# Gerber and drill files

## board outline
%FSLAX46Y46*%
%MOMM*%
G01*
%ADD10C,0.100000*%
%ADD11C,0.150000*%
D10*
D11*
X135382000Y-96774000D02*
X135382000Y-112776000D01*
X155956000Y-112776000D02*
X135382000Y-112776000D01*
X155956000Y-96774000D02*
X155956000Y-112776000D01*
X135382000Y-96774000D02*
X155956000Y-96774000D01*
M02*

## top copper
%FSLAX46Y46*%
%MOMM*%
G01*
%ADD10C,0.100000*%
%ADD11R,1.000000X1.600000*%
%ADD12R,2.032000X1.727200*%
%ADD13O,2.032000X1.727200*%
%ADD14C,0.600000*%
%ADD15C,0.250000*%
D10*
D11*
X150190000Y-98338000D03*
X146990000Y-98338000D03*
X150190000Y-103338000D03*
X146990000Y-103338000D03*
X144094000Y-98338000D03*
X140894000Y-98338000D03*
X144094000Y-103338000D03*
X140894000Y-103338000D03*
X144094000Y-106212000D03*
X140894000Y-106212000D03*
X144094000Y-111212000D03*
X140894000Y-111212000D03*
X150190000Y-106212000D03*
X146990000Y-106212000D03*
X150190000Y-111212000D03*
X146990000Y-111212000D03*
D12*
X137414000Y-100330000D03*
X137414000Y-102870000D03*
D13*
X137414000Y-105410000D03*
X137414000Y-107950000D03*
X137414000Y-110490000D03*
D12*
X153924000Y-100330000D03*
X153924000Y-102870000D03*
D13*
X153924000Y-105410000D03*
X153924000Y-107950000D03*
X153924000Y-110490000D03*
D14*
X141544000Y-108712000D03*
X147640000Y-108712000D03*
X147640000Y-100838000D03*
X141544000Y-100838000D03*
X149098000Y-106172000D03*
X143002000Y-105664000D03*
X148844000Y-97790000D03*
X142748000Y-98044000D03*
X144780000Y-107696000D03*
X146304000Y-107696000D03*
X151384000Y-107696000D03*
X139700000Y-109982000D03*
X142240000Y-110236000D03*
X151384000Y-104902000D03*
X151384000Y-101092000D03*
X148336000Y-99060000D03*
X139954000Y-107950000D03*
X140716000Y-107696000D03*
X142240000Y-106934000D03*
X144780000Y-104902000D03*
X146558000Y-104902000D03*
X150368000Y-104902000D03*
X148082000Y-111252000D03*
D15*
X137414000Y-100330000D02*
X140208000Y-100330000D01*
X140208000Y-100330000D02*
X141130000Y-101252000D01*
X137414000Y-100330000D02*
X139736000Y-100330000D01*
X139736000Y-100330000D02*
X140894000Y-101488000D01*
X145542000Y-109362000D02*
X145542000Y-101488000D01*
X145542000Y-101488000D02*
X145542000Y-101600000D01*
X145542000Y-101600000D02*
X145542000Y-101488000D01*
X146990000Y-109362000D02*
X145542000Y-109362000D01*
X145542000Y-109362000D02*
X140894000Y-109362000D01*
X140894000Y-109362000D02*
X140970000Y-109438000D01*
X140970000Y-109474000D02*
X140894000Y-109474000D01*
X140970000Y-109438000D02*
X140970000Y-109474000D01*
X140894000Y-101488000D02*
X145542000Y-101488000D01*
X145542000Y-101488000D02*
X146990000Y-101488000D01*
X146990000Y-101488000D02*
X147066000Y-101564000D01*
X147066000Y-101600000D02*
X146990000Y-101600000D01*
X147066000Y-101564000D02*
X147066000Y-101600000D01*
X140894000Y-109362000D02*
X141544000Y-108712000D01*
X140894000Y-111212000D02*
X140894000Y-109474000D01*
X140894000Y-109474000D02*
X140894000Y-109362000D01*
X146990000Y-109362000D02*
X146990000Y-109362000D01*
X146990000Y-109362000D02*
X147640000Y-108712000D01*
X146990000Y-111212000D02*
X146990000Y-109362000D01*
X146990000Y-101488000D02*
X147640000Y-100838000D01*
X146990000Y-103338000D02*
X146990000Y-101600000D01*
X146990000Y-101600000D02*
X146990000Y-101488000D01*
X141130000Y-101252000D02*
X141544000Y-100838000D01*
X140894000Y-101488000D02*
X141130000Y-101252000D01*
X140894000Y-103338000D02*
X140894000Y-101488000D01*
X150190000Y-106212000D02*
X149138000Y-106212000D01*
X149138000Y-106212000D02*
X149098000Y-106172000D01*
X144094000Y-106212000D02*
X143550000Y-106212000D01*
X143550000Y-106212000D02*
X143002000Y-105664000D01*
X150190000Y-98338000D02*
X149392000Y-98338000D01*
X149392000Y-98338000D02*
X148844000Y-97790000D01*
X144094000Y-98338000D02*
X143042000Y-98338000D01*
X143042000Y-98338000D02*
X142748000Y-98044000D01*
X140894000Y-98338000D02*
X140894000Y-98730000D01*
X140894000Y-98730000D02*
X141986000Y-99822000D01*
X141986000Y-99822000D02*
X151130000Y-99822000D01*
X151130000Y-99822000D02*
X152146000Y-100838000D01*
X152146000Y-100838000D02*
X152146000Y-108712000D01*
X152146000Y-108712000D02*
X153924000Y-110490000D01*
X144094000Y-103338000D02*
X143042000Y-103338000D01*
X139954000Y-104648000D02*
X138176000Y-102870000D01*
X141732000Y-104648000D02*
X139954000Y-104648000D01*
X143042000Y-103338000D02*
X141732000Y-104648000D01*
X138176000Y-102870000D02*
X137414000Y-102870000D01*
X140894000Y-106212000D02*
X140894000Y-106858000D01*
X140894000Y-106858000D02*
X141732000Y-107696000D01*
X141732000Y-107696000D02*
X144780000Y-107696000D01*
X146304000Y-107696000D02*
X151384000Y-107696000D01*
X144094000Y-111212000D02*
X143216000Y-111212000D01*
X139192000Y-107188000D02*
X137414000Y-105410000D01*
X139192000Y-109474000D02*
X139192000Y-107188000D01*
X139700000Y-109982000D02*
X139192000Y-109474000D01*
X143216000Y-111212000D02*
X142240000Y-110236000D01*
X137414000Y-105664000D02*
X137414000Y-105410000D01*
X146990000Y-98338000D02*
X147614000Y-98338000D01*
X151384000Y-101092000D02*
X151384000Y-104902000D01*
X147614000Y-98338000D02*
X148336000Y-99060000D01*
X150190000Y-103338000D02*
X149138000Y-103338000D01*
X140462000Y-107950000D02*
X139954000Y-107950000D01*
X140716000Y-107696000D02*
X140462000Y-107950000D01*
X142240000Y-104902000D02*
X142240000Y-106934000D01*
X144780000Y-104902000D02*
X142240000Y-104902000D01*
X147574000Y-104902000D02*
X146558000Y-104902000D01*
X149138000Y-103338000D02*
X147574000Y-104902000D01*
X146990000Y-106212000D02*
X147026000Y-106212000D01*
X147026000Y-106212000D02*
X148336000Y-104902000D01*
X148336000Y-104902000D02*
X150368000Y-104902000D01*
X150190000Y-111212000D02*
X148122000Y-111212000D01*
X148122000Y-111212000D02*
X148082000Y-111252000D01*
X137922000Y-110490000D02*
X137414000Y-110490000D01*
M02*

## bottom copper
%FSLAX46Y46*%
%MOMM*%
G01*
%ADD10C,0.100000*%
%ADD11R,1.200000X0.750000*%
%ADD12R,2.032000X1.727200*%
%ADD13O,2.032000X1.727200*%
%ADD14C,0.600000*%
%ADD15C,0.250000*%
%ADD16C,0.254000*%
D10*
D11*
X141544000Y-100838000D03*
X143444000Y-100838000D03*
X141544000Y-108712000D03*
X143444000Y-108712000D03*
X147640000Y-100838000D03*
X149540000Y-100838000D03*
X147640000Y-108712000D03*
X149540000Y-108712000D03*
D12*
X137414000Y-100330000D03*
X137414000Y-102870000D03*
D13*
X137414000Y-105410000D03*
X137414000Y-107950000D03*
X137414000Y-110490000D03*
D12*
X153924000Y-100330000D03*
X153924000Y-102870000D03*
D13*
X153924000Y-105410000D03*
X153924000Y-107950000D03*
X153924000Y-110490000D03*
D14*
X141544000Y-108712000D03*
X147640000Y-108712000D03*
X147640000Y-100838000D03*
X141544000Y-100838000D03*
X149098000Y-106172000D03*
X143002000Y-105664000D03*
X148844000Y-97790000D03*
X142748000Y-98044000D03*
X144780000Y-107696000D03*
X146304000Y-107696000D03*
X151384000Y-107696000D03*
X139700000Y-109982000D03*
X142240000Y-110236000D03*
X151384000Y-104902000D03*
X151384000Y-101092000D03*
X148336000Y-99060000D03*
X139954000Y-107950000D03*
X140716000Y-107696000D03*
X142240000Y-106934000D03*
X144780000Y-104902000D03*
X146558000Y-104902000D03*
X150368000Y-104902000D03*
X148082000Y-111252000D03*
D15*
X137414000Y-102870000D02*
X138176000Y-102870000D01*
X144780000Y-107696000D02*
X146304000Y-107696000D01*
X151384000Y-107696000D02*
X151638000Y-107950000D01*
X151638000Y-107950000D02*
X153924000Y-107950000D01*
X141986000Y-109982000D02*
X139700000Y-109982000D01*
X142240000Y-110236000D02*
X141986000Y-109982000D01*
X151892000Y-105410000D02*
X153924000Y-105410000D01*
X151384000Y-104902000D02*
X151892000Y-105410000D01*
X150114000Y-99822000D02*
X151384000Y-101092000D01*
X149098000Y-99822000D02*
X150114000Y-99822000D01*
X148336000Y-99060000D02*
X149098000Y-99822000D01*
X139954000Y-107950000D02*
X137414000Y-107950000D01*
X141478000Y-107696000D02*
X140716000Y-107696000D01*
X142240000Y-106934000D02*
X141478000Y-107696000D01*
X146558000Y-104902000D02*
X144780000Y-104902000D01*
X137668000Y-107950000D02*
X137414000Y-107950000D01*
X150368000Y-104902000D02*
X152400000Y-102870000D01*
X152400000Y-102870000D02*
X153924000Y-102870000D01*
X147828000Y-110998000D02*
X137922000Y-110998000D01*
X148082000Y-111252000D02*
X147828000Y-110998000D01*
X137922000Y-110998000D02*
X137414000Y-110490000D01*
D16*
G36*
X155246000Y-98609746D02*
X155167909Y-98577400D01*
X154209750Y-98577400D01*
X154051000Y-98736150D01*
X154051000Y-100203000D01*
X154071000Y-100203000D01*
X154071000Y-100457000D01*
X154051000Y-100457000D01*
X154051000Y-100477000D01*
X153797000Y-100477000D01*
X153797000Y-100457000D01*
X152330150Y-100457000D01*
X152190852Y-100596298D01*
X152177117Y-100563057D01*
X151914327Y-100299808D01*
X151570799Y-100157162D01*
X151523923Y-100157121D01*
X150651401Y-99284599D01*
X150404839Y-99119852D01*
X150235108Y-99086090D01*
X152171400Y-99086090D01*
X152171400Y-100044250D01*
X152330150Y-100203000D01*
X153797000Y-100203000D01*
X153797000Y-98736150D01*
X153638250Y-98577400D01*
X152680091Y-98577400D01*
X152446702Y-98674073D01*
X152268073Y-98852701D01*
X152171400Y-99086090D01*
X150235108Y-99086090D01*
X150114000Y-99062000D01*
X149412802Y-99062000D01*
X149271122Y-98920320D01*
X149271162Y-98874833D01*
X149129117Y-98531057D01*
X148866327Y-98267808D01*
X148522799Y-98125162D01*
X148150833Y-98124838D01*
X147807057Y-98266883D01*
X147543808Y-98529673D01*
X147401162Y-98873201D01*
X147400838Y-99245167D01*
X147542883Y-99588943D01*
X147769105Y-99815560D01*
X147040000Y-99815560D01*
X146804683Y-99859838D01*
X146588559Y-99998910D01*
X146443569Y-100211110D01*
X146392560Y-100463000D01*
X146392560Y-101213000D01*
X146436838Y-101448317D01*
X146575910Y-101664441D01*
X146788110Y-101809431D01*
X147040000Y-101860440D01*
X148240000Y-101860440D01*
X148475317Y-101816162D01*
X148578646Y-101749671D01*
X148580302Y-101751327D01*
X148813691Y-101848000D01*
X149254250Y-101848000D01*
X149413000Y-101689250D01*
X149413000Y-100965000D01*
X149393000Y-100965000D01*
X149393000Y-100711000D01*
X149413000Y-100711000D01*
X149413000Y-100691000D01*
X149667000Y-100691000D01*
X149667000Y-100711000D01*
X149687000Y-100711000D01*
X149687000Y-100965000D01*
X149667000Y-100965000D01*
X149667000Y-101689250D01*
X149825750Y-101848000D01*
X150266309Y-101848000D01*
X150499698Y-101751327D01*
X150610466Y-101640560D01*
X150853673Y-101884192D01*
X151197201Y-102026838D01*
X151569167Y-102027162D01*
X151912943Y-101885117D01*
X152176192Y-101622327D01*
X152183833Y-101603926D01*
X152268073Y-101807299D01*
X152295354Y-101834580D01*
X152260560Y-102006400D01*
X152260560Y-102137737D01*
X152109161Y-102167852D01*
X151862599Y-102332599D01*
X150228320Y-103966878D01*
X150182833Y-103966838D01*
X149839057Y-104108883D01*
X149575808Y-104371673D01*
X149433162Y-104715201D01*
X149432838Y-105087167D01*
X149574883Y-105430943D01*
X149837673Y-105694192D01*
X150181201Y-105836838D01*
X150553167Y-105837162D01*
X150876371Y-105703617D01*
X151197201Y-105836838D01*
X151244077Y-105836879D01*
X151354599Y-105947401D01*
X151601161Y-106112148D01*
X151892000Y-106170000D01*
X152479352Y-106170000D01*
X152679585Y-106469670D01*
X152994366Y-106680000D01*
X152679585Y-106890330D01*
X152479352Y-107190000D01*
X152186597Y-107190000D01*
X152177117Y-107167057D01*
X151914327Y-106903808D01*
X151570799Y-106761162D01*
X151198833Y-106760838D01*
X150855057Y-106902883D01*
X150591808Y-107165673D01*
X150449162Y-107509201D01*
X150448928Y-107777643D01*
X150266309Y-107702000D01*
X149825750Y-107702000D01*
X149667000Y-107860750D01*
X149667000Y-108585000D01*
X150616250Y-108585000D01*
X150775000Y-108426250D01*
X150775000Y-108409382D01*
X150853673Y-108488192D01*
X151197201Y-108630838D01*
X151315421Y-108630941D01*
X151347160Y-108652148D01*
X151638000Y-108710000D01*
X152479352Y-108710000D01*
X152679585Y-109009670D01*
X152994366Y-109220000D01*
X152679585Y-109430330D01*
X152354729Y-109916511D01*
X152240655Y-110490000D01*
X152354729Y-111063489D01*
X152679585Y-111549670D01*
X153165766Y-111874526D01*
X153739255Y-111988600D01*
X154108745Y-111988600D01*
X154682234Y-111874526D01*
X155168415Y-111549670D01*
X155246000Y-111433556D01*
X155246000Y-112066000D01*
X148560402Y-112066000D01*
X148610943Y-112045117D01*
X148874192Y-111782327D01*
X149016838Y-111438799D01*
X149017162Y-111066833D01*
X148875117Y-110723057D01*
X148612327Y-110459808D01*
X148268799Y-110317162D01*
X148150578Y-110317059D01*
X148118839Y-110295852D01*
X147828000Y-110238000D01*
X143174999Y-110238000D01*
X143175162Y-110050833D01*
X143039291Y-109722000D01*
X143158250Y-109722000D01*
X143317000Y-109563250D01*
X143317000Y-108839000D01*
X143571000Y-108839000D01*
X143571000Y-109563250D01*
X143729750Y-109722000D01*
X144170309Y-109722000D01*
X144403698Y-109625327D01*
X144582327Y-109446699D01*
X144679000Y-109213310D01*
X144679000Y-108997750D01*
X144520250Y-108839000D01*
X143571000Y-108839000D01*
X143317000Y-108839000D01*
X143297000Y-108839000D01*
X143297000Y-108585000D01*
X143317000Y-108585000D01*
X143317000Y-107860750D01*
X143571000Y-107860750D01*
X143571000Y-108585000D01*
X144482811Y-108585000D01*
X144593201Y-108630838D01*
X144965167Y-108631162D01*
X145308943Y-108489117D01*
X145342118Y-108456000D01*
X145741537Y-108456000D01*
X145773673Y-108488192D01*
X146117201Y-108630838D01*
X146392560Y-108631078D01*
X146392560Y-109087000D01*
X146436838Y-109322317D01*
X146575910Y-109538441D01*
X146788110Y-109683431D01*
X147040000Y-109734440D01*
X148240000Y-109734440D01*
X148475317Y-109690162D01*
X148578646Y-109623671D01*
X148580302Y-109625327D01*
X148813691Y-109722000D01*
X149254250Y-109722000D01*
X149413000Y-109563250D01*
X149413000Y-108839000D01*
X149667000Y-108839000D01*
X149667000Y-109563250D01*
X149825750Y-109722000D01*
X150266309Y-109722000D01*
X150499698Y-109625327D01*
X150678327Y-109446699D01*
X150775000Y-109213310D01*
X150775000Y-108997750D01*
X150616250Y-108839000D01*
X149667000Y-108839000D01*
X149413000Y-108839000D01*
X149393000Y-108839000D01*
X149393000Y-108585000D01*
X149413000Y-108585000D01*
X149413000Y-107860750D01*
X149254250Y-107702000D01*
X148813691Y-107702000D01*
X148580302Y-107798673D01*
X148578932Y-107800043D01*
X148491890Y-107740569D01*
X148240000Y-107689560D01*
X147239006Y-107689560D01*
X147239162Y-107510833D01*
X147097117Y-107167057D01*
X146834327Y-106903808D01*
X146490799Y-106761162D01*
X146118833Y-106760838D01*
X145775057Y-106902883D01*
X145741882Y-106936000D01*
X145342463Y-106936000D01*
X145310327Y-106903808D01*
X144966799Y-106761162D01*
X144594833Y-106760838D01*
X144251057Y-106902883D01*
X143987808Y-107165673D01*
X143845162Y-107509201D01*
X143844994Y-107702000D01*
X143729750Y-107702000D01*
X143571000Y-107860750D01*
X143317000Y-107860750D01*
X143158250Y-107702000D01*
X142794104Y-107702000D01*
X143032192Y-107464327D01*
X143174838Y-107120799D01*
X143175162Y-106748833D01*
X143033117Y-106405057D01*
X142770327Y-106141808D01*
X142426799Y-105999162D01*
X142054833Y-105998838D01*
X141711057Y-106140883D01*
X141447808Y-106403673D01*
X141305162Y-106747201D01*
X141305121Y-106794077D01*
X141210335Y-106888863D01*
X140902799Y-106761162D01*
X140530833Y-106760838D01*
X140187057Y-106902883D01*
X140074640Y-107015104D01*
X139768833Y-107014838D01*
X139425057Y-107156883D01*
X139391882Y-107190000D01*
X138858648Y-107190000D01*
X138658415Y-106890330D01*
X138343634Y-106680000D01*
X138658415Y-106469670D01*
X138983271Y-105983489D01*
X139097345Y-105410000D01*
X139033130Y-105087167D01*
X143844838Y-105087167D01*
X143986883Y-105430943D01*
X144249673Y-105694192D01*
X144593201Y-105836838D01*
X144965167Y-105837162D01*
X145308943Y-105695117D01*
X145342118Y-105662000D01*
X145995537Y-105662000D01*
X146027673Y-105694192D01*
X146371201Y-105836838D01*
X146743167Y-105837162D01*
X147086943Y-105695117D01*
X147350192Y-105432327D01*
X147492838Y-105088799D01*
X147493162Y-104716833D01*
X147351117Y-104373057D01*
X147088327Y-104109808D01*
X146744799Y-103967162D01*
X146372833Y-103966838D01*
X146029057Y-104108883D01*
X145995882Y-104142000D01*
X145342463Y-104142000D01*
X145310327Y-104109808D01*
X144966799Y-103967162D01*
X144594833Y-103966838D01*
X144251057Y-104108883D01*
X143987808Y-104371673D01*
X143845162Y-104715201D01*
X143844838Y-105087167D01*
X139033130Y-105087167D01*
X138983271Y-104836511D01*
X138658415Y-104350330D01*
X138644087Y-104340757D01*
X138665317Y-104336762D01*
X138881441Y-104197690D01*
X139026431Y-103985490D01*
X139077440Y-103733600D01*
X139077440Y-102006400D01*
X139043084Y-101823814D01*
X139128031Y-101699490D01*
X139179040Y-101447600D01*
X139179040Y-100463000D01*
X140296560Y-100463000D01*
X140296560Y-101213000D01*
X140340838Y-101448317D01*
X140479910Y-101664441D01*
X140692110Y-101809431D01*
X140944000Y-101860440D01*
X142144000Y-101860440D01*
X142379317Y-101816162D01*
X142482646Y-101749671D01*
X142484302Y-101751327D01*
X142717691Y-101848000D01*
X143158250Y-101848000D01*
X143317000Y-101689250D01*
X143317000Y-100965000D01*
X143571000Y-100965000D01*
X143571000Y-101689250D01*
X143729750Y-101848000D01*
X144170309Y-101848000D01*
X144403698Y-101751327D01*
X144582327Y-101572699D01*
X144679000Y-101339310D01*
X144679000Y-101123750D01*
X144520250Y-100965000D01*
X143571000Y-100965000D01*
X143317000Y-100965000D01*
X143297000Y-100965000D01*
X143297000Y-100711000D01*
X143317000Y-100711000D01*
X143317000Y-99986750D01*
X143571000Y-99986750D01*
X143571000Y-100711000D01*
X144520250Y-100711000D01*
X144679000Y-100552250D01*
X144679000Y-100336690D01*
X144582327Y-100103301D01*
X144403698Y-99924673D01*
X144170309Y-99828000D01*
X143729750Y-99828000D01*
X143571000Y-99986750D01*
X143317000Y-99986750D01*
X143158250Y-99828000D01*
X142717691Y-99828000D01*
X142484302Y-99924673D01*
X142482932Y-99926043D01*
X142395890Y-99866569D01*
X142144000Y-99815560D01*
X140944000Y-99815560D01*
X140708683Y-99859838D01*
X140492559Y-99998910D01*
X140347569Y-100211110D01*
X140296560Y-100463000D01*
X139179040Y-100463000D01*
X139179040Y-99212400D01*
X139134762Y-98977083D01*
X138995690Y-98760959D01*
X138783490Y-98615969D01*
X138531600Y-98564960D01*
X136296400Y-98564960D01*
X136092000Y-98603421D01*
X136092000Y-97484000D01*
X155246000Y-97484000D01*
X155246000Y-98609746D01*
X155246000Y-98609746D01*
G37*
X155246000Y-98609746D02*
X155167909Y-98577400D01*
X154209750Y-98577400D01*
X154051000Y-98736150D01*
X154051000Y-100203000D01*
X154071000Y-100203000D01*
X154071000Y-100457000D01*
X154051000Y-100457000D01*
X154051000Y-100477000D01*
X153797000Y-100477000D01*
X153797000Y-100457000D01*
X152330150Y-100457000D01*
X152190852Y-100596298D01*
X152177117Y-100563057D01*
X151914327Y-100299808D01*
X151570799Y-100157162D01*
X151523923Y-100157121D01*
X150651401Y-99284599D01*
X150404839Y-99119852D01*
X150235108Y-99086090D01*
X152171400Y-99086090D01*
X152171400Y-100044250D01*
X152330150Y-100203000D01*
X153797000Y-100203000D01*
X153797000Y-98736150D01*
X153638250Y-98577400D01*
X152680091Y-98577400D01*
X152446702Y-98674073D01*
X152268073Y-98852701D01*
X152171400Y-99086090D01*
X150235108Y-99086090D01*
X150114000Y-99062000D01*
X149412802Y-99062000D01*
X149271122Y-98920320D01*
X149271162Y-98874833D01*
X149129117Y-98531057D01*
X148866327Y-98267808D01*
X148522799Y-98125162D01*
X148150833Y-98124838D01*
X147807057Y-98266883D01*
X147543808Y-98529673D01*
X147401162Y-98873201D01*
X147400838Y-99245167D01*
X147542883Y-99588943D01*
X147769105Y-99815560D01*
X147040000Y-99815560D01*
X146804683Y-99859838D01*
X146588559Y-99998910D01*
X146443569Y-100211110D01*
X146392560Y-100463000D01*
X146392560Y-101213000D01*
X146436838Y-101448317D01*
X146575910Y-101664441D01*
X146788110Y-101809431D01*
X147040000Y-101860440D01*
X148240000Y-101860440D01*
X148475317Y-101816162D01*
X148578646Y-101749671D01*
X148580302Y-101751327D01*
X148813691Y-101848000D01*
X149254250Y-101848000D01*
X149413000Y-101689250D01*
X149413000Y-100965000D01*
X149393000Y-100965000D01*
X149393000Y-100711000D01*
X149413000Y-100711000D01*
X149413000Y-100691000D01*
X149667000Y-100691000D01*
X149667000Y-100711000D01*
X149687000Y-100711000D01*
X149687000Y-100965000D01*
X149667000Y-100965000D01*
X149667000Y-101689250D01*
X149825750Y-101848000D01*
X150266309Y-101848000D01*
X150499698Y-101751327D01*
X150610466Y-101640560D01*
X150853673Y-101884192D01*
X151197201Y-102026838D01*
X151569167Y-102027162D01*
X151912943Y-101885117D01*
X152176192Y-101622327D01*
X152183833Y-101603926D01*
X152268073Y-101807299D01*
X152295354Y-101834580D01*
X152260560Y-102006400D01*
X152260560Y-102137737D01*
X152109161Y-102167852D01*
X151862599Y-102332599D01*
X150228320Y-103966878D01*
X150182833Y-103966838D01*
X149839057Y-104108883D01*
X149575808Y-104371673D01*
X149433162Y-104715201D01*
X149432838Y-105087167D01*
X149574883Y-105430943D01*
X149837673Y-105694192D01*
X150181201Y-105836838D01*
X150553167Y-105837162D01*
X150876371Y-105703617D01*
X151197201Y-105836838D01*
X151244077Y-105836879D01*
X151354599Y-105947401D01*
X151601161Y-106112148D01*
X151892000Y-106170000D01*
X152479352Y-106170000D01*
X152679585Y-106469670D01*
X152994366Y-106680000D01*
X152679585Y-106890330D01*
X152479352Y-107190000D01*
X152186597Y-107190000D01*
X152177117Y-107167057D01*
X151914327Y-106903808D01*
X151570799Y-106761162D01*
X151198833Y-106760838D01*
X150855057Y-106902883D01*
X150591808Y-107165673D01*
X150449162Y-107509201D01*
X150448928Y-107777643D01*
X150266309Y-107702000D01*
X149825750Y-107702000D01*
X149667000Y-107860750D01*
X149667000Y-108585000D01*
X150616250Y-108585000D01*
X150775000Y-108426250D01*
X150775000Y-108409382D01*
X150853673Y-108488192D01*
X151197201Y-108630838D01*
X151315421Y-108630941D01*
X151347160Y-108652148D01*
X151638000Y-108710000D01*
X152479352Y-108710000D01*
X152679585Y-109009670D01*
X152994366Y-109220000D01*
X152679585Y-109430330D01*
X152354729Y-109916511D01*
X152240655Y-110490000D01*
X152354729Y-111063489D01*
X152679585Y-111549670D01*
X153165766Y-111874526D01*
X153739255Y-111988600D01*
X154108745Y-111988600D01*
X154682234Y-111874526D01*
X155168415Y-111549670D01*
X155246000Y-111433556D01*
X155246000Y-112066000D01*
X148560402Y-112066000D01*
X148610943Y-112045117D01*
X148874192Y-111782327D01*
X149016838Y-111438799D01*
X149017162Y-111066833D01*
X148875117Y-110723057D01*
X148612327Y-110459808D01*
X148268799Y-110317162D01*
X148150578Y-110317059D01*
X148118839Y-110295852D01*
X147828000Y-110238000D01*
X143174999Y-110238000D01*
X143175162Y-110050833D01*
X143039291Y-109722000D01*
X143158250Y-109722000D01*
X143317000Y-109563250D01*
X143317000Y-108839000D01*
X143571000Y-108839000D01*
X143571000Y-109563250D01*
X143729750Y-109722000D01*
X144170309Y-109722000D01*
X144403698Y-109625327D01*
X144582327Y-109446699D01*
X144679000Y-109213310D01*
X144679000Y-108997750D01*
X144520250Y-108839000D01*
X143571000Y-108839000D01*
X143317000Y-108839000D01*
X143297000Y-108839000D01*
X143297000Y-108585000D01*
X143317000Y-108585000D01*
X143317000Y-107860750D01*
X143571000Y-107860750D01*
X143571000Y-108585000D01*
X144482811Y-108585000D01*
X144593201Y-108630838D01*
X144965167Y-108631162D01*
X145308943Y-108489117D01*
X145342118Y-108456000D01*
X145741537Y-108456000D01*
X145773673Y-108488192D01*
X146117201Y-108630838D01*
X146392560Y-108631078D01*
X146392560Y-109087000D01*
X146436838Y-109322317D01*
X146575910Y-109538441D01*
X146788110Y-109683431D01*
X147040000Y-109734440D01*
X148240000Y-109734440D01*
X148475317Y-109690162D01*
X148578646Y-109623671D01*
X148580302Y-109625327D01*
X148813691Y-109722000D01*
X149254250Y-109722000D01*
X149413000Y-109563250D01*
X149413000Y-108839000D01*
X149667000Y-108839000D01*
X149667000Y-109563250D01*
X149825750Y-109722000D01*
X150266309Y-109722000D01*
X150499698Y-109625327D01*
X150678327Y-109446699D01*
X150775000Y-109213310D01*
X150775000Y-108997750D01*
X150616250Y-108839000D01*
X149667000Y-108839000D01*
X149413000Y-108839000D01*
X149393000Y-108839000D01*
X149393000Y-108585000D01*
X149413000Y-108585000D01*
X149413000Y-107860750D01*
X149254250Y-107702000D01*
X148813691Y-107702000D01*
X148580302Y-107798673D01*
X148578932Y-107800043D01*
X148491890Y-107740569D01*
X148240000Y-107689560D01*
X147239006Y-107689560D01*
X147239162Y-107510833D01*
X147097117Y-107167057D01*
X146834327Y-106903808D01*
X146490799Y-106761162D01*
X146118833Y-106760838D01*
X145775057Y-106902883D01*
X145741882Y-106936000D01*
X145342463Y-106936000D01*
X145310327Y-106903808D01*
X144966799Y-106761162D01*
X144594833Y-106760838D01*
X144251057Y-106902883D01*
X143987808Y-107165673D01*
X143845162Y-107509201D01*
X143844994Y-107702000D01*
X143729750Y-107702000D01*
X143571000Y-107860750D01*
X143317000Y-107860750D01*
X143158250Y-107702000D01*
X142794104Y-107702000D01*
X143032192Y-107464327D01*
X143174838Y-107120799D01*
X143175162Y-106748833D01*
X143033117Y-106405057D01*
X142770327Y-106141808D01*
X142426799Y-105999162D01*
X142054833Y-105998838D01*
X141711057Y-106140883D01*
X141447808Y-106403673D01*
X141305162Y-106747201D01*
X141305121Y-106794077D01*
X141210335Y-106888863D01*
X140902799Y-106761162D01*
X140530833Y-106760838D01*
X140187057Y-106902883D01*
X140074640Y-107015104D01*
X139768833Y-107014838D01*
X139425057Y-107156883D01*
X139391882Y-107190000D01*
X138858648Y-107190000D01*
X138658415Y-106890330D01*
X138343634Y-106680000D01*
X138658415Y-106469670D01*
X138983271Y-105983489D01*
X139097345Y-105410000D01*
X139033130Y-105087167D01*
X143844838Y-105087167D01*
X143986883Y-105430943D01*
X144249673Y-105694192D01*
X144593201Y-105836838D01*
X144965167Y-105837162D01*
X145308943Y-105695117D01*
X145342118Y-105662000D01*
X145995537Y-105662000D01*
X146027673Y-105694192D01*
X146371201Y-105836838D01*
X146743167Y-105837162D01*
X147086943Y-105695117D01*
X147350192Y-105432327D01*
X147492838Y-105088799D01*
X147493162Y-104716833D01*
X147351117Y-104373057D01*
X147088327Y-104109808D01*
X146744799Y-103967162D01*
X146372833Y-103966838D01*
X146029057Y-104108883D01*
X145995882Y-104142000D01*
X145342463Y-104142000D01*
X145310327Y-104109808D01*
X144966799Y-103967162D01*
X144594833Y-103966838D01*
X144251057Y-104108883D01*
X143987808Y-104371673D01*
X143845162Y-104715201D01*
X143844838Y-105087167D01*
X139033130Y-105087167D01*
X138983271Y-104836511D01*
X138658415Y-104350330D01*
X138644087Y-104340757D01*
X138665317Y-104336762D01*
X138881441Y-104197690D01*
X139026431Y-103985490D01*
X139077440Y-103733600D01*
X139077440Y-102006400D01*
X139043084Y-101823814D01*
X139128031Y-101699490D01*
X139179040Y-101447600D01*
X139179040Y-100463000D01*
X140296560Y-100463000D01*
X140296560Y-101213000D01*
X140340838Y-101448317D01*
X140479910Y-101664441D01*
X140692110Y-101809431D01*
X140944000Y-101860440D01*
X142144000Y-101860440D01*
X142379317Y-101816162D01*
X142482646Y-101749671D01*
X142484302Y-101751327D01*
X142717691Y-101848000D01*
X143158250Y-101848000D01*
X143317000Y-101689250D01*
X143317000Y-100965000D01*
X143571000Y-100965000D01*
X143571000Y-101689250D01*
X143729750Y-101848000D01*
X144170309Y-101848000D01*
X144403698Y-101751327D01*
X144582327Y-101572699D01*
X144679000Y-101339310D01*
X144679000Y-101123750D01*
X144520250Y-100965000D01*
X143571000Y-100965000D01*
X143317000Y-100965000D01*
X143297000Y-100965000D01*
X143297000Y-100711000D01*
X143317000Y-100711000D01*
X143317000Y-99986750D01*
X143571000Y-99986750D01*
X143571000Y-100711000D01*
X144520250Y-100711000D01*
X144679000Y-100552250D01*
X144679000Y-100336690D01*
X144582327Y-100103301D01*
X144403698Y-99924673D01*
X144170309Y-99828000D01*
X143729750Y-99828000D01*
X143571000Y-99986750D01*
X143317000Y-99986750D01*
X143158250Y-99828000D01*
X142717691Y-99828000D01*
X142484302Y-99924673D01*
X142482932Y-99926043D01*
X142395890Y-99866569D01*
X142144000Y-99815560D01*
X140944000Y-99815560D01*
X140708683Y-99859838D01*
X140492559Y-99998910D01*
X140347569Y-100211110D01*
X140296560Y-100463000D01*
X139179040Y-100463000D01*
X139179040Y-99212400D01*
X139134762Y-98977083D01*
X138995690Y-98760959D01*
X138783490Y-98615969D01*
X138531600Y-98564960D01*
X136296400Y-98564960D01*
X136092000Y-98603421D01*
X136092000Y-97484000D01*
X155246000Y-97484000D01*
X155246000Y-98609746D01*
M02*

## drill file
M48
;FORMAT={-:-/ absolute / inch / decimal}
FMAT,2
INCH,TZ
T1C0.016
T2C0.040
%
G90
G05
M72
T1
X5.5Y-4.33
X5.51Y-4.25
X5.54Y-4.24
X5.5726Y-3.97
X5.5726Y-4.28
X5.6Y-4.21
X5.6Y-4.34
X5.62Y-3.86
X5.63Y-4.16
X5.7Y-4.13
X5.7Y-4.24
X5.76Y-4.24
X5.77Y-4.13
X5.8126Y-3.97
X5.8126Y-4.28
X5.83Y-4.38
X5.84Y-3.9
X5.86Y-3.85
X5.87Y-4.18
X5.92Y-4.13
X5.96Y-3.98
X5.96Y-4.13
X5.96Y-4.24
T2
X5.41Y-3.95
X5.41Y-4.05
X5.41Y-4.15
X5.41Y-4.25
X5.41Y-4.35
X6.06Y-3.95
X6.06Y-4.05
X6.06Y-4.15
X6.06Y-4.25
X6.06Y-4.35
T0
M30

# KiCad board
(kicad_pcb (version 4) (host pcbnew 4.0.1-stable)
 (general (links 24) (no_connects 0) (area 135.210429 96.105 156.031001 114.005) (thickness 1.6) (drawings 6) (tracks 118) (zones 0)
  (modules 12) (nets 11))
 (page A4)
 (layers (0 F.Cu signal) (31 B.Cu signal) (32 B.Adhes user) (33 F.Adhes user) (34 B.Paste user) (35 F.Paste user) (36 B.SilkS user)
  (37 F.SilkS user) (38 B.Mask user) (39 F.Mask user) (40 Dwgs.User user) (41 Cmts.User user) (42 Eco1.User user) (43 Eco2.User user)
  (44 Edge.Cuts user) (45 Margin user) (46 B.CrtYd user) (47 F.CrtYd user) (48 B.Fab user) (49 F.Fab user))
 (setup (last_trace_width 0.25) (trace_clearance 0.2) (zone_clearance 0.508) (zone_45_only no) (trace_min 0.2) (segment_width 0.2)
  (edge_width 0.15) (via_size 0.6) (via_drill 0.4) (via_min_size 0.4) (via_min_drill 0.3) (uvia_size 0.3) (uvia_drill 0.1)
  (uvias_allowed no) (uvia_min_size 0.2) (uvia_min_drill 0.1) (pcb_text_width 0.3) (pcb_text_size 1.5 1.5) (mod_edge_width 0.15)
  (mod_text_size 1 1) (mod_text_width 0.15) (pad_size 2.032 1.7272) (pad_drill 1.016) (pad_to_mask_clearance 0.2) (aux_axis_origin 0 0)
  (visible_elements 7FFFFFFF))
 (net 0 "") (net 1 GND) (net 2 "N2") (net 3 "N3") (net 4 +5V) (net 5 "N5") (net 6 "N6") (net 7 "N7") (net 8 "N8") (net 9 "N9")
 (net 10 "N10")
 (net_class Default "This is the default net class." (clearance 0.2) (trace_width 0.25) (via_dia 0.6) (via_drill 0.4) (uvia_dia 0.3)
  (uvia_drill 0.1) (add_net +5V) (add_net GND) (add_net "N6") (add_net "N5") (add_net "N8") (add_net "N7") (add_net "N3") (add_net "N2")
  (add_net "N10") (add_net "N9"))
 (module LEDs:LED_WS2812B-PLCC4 (layer F.Cu) (at 148.59 100.838 90)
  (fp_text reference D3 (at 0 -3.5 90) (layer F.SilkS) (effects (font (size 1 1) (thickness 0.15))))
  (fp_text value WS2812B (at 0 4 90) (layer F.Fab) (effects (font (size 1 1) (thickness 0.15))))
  (pad 3 smd rect (at 2.5 1.6 90) (size 1.6 1) (layers F.Cu F.Paste F.Mask) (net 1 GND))
  (pad 4 smd rect (at 2.5 -1.6 90) (size 1.6 1) (layers F.Cu F.Paste F.Mask) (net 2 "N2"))
  (pad 2 smd rect (at -2.5 1.6 90) (size 1.6 1) (layers F.Cu F.Paste F.Mask) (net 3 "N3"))
  (pad 1 smd rect (at -2.5 -1.6 90) (size 1.6 1) (layers F.Cu F.Paste F.Mask) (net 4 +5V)))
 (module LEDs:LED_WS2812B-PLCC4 (layer F.Cu) (at 142.494 100.838 90)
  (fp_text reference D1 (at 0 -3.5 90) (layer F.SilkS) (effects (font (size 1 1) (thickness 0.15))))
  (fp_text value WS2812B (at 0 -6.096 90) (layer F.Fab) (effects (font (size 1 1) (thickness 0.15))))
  (pad 3 smd rect (at 2.5 1.6 90) (size 1.6 1) (layers F.Cu F.Paste F.Mask) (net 1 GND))
  (pad 4 smd rect (at 2.5 -1.6 90) (size 1.6 1) (layers F.Cu F.Paste F.Mask) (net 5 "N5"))
  (pad 2 smd rect (at -2.5 1.6 90) (size 1.6 1) (layers F.Cu F.Paste F.Mask) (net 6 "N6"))
  (pad 1 smd rect (at -2.5 -1.6 90) (size 1.6 1) (layers F.Cu F.Paste F.Mask) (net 4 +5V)))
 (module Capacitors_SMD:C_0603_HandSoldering (layer B.Cu) (at 142.494 100.838)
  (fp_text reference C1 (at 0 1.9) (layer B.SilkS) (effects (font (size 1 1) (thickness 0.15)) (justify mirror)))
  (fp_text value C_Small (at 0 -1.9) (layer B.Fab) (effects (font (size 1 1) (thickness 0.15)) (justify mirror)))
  (pad 1 smd rect (at -0.95 0) (size 1.2 0.75) (layers B.Cu B.Paste B.Mask) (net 4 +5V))
  (pad 2 smd rect (at 0.95 0) (size 1.2 0.75) (layers B.Cu B.Paste B.Mask) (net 1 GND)))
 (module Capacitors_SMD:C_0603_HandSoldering (layer B.Cu) (at 142.494 108.712)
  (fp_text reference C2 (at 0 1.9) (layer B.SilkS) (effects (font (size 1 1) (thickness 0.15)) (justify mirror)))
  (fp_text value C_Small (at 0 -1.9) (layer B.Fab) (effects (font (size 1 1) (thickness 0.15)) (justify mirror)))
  (pad 1 smd rect (at -0.95 0) (size 1.2 0.75) (layers B.Cu B.Paste B.Mask) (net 4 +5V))
  (pad 2 smd rect (at 0.95 0) (size 1.2 0.75) (layers B.Cu B.Paste B.Mask) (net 1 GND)))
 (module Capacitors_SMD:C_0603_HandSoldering (layer B.Cu) (at 148.59 100.838)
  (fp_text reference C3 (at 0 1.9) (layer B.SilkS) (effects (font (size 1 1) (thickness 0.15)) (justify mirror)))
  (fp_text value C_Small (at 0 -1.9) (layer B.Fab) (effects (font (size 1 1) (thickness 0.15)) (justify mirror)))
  (pad 1 smd rect (at -0.95 0) (size 1.2 0.75) (layers B.Cu B.Paste B.Mask) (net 4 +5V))
  (pad 2 smd rect (at 0.95 0) (size 1.2 0.75) (layers B.Cu B.Paste B.Mask) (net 1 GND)))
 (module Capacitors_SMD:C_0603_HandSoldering (layer B.Cu) (at 148.59 108.712)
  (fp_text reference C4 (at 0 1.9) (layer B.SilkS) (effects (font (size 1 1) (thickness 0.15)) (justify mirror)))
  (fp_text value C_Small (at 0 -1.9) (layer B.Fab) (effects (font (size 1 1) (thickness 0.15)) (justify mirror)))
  (pad 1 smd rect (at -0.95 0) (size 1.2 0.75) (layers B.Cu B.Paste B.Mask) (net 4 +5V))
  (pad 2 smd rect (at 0.95 0) (size 1.2 0.75) (layers B.Cu B.Paste B.Mask) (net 1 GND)))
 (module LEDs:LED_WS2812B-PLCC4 (layer F.Cu) (at 142.494 108.712 90)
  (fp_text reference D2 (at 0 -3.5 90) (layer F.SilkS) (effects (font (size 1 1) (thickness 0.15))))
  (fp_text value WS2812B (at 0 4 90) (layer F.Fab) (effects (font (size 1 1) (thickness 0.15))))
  (pad 3 smd rect (at 2.5 1.6 90) (size 1.6 1) (layers F.Cu F.Paste F.Mask) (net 1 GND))
  (pad 4 smd rect (at 2.5 -1.6 90) (size 1.6 1) (layers F.Cu F.Paste F.Mask) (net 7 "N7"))
  (pad 2 smd rect (at -2.5 1.6 90) (size 1.6 1) (layers F.Cu F.Paste F.Mask) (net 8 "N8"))
  (pad 1 smd rect (at -2.5 -1.6 90) (size 1.6 1) (layers F.Cu F.Paste F.Mask) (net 4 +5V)))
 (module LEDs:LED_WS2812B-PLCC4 (layer F.Cu) (at 148.59 108.712 90)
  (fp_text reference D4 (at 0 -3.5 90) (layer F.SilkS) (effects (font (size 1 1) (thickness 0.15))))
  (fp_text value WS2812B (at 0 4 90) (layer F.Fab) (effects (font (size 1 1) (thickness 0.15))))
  (pad 3 smd rect (at 2.5 1.6 90) (size 1.6 1) (layers F.Cu F.Paste F.Mask) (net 1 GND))
  (pad 4 smd rect (at 2.5 -1.6 90) (size 1.6 1) (layers F.Cu F.Paste F.Mask) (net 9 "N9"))
  (pad 2 smd rect (at -2.5 1.6 90) (size 1.6 1) (layers F.Cu F.Paste F.Mask) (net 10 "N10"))
  (pad 1 smd rect (at -2.5 -1.6 90) (size 1.6 1) (layers F.Cu F.Paste F.Mask) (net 4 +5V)))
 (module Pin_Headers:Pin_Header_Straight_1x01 (layer F.Cu) (at 137.414 100.33)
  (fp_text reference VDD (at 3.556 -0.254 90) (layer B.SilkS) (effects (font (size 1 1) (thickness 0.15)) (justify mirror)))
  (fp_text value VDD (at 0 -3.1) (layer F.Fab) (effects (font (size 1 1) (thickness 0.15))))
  (pad 1 thru_hole rect (at 0 0) (size 2.032 1.7272) (drill 1.016) (layers *.Cu *.Mask F.SilkS) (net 4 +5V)))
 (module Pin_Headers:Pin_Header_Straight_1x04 (layer F.Cu) (at 137.414 102.87)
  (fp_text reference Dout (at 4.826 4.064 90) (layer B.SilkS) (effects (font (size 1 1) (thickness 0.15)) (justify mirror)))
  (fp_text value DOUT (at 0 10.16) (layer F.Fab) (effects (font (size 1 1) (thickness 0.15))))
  (pad 1 thru_hole rect (at 0 0) (size 2.032 1.7272) (drill 1.016) (layers *.Cu *.Mask F.SilkS) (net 6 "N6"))
  (pad 2 thru_hole oval (at 0 2.54) (size 2.032 1.7272) (drill 1.016) (layers *.Cu *.Mask F.SilkS) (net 8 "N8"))
  (pad 3 thru_hole oval (at 0 5.08) (size 2.032 1.7272) (drill 1.016) (layers *.Cu *.Mask F.SilkS) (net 3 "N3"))
  (pad 4 thru_hole oval (at 0 7.62) (size 2.032 1.7272) (drill 1.016) (layers *.Cu *.Mask F.SilkS) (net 10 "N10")))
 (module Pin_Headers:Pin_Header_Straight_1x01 (layer F.Cu) (at 153.924 100.33)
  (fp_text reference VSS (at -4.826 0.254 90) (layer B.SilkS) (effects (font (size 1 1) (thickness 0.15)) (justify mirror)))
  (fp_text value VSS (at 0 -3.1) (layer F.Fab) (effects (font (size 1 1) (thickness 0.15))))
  (pad 1 thru_hole rect (at 0 0) (size 2.032 1.7272) (drill 1.016) (layers *.Cu *.Mask F.SilkS) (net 1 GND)))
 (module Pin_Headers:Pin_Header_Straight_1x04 (layer F.Cu) (at 153.924 102.87)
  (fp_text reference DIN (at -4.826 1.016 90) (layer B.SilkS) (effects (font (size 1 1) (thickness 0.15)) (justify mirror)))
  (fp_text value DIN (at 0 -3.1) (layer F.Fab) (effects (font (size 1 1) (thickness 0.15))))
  (pad 1 thru_hole rect (at 0 0) (size 2.032 1.7272) (drill 1.016) (layers *.Cu *.Mask F.SilkS) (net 9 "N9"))
  (pad 2 thru_hole oval (at 0 2.54) (size 2.032 1.7272) (drill 1.016) (layers *.Cu *.Mask F.SilkS) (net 2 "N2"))
  (pad 3 thru_hole oval (at 0 5.08) (size 2.032 1.7272) (drill 1.016) (layers *.Cu *.Mask F.SilkS) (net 7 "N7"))
  (pad 4 thru_hole oval (at 0 7.62) (size 2.032 1.7272) (drill 1.016) (layers *.Cu *.Mask F.SilkS) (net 5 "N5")))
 (gr_line (start 135.382 96.774) (end 135.382 112.776) (angle 90) (layer Edge.Cuts) (width 0.15))
 (gr_line (start 155.956 112.776) (end 135.382 112.776) (angle 90) (layer Edge.Cuts) (width 0.15))
 (gr_line (start 155.956 96.774) (end 155.956 112.776) (angle 90) (layer Edge.Cuts) (width 0.15))
 (gr_line (start 135.382 96.774) (end 155.956 96.774) (angle 90) (layer Edge.Cuts) (width 0.15))
 (segment (start 137.414 100.33) (end 140.208 100.33) (width 0.25) (layer F.Cu) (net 4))
 (segment (start 140.208 100.33) (end 141.13 101.252) (width 0.25) (layer F.Cu) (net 4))
 (segment (start 137.414 100.33) (end 139.736 100.33) (width 0.25) (layer F.Cu) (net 4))
 (segment (start 139.736 100.33) (end 140.894 101.488) (width 0.25) (layer F.Cu) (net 4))
 (segment (start 145.542 109.362) (end 145.542 101.488) (width 0.25) (layer F.Cu) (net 4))
 (segment (start 145.542 101.488) (end 145.542 101.6) (width 0.25) (layer F.Cu) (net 4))
 (segment (start 145.542 101.6) (end 145.542 101.488) (width 0.25) (layer F.Cu) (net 4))
 (segment (start 146.99 109.362) (end 145.542 109.362) (width 0.25) (layer F.Cu) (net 4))
 (segment (start 145.542 109.362) (end 140.894 109.362) (width 0.25) (layer F.Cu) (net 4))
 (segment (start 140.894 109.362) (end 140.97 109.438) (width 0.25) (layer F.Cu) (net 4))
 (segment (start 140.97 109.474) (end 140.894 109.474) (width 0.25) (layer F.Cu) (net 4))
 (segment (start 140.97 109.438) (end 140.97 109.474) (width 0.25) (layer F.Cu) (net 4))
 (segment (start 140.894 101.488) (end 145.542 101.488) (width 0.25) (layer F.Cu) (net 4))
 (segment (start 145.542 101.488) (end 146.99 101.488) (width 0.25) (layer F.Cu) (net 4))
 (segment (start 146.99 101.488) (end 147.066 101.564) (width 0.25) (layer F.Cu) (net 4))
 (segment (start 147.066 101.6) (end 146.99 101.6) (width 0.25) (layer F.Cu) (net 4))
 (segment (start 147.066 101.564) (end 147.066 101.6) (width 0.25) (layer F.Cu) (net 4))
 (via (at 141.544 108.712) (size 0.6) (drill 0.4) (layers F.Cu B.Cu) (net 4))
 (segment (start 140.894 109.362) (end 141.544 108.712) (width 0.25) (layer F.Cu) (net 4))
 (segment (start 140.894 111.212) (end 140.894 109.474) (width 0.25) (layer F.Cu) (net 4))
 (segment (start 140.894 109.474) (end 140.894 109.362) (width 0.25) (layer F.Cu) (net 4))
 (via (at 147.64 108.712) (size 0.6) (drill 0.4) (layers F.Cu B.Cu) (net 4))
 (segment (start 146.99 109.362) (end 146.99 109.362) (width 0.25) (layer F.Cu) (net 4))
 (segment (start 146.99 109.362) (end 147.64 108.712) (width 0.25) (layer F.Cu) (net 4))
 (segment (start 146.99 111.212) (end 146.99 109.362) (width 0.25) (layer F.Cu) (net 4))
 (via (at 147.64 100.838) (size 0.6) (drill 0.4) (layers F.Cu B.Cu) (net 4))
 (segment (start 146.99 101.488) (end 147.64 100.838) (width 0.25) (layer F.Cu) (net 4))
 (segment (start 146.99 103.338) (end 146.99 101.6) (width 0.25) (layer F.Cu) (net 4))
 (segment (start 146.99 101.6) (end 146.99 101.488) (width 0.25) (layer F.Cu) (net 4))
 (via (at 141.544 100.838) (size 0.6) (drill 0.4) (layers F.Cu B.Cu) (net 4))
 (segment (start 141.13 101.252) (end 141.544 100.838) (width 0.25) (layer F.Cu) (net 4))
 (segment (start 140.894 101.488) (end 141.13 101.252) (width 0.25) (layer F.Cu) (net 4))
 (segment (start 140.894 103.338) (end 140.894 101.488) (width 0.25) (layer F.Cu) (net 4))
 (segment (start 150.19 106.212) (end 149.138 106.212) (width 0.25) (layer F.Cu) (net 1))
 (via (at 149.098 106.172) (size 0.6) (drill 0.4) (layers F.Cu B.Cu) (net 1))
 (segment (start 149.138 106.212) (end 149.098 106.172) (width 0.25) (layer F.Cu) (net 1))
 (segment (start 144.094 106.212) (end 143.55 106.212) (width 0.25) (layer F.Cu) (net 1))
 (via (at 143.002 105.664) (size 0.6) (drill 0.4) (layers F.Cu B.Cu) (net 1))
 (segment (start 143.55 106.212) (end 143.002 105.664) (width 0.25) (layer F.Cu) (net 1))
 (segment (start 150.19 98.338) (end 149.392 98.338) (width 0.25) (layer F.Cu) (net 1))
 (via (at 148.844 97.79) (size 0.6) (drill 0.4) (layers F.Cu B.Cu) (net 1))
 (segment (start 149.392 98.338) (end 148.844 97.79) (width 0.25) (layer F.Cu) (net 1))
 (segment (start 144.094 98.338) (end 143.042 98.338) (width 0.25) (layer F.Cu) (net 1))
 (via (at 142.748 98.044) (size 0.6) (drill 0.4) (layers F.Cu B.Cu) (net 1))
 (segment (start 143.042 98.338) (end 142.748 98.044) (width 0.25) (layer F.Cu) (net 1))
 (segment (start 140.894 98.338) (end 140.894 98.73) (width 0.25) (layer F.Cu) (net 5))
 (segment (start 140.894 98.73) (end 141.986 99.822) (width 0.25) (layer F.Cu) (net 5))
 (segment (start 141.986 99.822) (end 151.13 99.822) (width 0.25) (layer F.Cu) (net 5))
 (segment (start 151.13 99.822) (end 152.146 100.838) (width 0.25) (layer F.Cu) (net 5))
 (segment (start 152.146 100.838) (end 152.146 108.712) (width 0.25) (layer F.Cu) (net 5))
 (segment (start 152.146 108.712) (end 153.924 110.49) (width 0.25) (layer F.Cu) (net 5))
 (segment (start 144.094 103.338) (end 143.042 103.338) (width 0.25) (layer F.Cu) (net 6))
 (segment (start 139.954 104.648) (end 138.176 102.87) (width 0.25) (layer F.Cu) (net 6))
 (segment (start 141.732 104.648) (end 139.954 104.648) (width 0.25) (layer F.Cu) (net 6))
 (segment (start 143.042 103.338) (end 141.732 104.648) (width 0.25) (layer F.Cu) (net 6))
 (segment (start 138.176 102.87) (end 137.414 102.87) (width 0.25) (layer F.Cu) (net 6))
 (segment (start 137.414 102.87) (end 138.176 102.87) (width 0.25) (layer B.Cu) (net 6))
 (segment (start 140.894 106.212) (end 140.894 106.858) (width 0.25) (layer F.Cu) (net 7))
 (segment (start 140.894 106.858) (end 141.732 107.696) (width 0.25) (layer F.Cu) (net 7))
 (segment (start 141.732 107.696) (end 144.78 107.696) (width 0.25) (layer F.Cu) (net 7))
 (via (at 144.78 107.696) (size 0.6) (drill 0.4) (layers F.Cu B.Cu) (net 7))
 (segment (start 144.78 107.696) (end 146.304 107.696) (width 0.25) (layer B.Cu) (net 7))
 (via (at 146.304 107.696) (size 0.6) (drill 0.4) (layers F.Cu B.Cu) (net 7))
 (segment (start 146.304 107.696) (end 151.384 107.696) (width 0.25) (layer F.Cu) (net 7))
 (via (at 151.384 107.696) (size 0.6) (drill 0.4) (layers F.Cu B.Cu) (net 7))
 (segment (start 151.384 107.696) (end 151.638 107.95) (width 0.25) (layer B.Cu) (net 7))
 (segment (start 151.638 107.95) (end 153.924 107.95) (width 0.25) (layer B.Cu) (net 7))
 (segment (start 144.094 111.212) (end 143.216 111.212) (width 0.25) (layer F.Cu) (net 8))
 (segment (start 139.192 107.188) (end 137.414 105.41) (width 0.25) (layer F.Cu) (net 8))
 (segment (start 139.192 109.474) (end 139.192 107.188) (width 0.25) (layer F.Cu) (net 8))
 (segment (start 139.7 109.982) (end 139.192 109.474) (width 0.25) (layer F.Cu) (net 8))
 (via (at 139.7 109.982) (size 0.6) (drill 0.4) (layers F.Cu B.Cu) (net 8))
 (segment (start 141.986 109.982) (end 139.7 109.982) (width 0.25) (layer B.Cu) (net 8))
 (segment (start 142.24 110.236) (end 141.986 109.982) (width 0.25) (layer B.Cu) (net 8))
 (via (at 142.24 110.236) (size 0.6) (drill 0.4) (layers F.Cu B.Cu) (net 8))
 (segment (start 143.216 111.212) (end 142.24 110.236) (width 0.25) (layer F.Cu) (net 8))
 (segment (start 137.414 105.664) (end 137.414 105.41) (width 0.25) (layer F.Cu) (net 8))
 (segment (start 146.99 98.338) (end 147.614 98.338) (width 0.25) (layer F.Cu) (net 2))
 (segment (start 151.892 105.41) (end 153.924 105.41) (width 0.25) (layer B.Cu) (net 2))
 (segment (start 151.384 104.902) (end 151.892 105.41) (width 0.25) (layer B.Cu) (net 2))
 (via (at 151.384 104.902) (size 0.6) (drill 0.4) (layers F.Cu B.Cu) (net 2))
 (segment (start 151.384 101.092) (end 151.384 104.902) (width 0.25) (layer F.Cu) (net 2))
 (via (at 151.384 101.092) (size 0.6) (drill 0.4) (layers F.Cu B.Cu) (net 2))
 (segment (start 150.114 99.822) (end 151.384 101.092) (width 0.25) (layer B.Cu) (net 2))
 (segment (start 149.098 99.822) (end 150.114 99.822) (width 0.25) (layer B.Cu) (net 2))
 (segment (start 148.336 99.06) (end 149.098 99.822) (width 0.25) (layer B.Cu) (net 2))
 (via (at 148.336 99.06) (size 0.6) (drill 0.4) (layers F.Cu B.Cu) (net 2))
 (segment (start 147.614 98.338) (end 148.336 99.06) (width 0.25) (layer F.Cu) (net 2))
 (segment (start 150.19 103.338) (end 149.138 103.338) (width 0.25) (layer F.Cu) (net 3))
 (segment (start 139.954 107.95) (end 137.414 107.95) (width 0.25) (layer B.Cu) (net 3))
 (via (at 139.954 107.95) (size 0.6) (drill 0.4) (layers F.Cu B.Cu) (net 3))
 (segment (start 140.462 107.95) (end 139.954 107.95) (width 0.25) (layer F.Cu) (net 3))
 (segment (start 140.716 107.696) (end 140.462 107.95) (width 0.25) (layer F.Cu) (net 3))
 (via (at 140.716 107.696) (size 0.6) (drill 0.4) (layers F.Cu B.Cu) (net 3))
 (segment (start 141.478 107.696) (end 140.716 107.696) (width 0.25) (layer B.Cu) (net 3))
 (segment (start 142.24 106.934) (end 141.478 107.696) (width 0.25) (layer B.Cu) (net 3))
 (via (at 142.24 106.934) (size 0.6) (drill 0.4) (layers F.Cu B.Cu) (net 3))
 (segment (start 142.24 104.902) (end 142.24 106.934) (width 0.25) (layer F.Cu) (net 3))
 (segment (start 144.78 104.902) (end 142.24 104.902) (width 0.25) (layer F.Cu) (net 3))
 (via (at 144.78 104.902) (size 0.6) (drill 0.4) (layers F.Cu B.Cu) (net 3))
 (segment (start 146.558 104.902) (end 144.78 104.902) (width 0.25) (layer B.Cu) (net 3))
 (via (at 146.558 104.902) (size 0.6) (drill 0.4) (layers F.Cu B.Cu) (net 3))
 (segment (start 147.574 104.902) (end 146.558 104.902) (width 0.25) (layer F.Cu) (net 3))
 (segment (start 149.138 103.338) (end 147.574 104.902) (width 0.25) (layer F.Cu) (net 3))
 (segment (start 137.668 107.95) (end 137.414 107.95) (width 0.25) (layer B.Cu) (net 3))
 (segment (start 146.99 106.212) (end 147.026 106.212) (width 0.25) (layer F.Cu) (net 9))
 (segment (start 147.026 106.212) (end 148.336 104.902) (width 0.25) (layer F.Cu) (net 9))
 (segment (start 148.336 104.902) (end 150.368 104.902) (width 0.25) (layer F.Cu) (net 9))
 (via (at 150.368 104.902) (size 0.6) (drill 0.4) (layers F.Cu B.Cu) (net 9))
 (segment (start 150.368 104.902) (end 152.4 102.87) (width 0.25) (layer B.Cu) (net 9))
 (segment (start 152.4 102.87) (end 153.924 102.87) (width 0.25) (layer B.Cu) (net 9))
 (segment (start 150.19 111.212) (end 148.122 111.212) (width 0.25) (layer F.Cu) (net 10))
 (segment (start 147.828 110.998) (end 137.922 110.998) (width 0.25) (layer B.Cu) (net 10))
 (segment (start 148.082 111.252) (end 147.828 110.998) (width 0.25) (layer B.Cu) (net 10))
 (via (at 148.082 111.252) (size 0.6) (drill 0.4) (layers F.Cu B.Cu) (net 10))
 (segment (start 148.122 111.212) (end 148.082 111.252) (width 0.25) (layer F.Cu) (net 10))
 (segment (start 137.922 110.998) (end 137.414 110.49) (width 0.25) (layer B.Cu) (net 10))
 (segment (start 137.922 110.49) (end 137.414 110.49) (width 0.25) (layer F.Cu) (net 10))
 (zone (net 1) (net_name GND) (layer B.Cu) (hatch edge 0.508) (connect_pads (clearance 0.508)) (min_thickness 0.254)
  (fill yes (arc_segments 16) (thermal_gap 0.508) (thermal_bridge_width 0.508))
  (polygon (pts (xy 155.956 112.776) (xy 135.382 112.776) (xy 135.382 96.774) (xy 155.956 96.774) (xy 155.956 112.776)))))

